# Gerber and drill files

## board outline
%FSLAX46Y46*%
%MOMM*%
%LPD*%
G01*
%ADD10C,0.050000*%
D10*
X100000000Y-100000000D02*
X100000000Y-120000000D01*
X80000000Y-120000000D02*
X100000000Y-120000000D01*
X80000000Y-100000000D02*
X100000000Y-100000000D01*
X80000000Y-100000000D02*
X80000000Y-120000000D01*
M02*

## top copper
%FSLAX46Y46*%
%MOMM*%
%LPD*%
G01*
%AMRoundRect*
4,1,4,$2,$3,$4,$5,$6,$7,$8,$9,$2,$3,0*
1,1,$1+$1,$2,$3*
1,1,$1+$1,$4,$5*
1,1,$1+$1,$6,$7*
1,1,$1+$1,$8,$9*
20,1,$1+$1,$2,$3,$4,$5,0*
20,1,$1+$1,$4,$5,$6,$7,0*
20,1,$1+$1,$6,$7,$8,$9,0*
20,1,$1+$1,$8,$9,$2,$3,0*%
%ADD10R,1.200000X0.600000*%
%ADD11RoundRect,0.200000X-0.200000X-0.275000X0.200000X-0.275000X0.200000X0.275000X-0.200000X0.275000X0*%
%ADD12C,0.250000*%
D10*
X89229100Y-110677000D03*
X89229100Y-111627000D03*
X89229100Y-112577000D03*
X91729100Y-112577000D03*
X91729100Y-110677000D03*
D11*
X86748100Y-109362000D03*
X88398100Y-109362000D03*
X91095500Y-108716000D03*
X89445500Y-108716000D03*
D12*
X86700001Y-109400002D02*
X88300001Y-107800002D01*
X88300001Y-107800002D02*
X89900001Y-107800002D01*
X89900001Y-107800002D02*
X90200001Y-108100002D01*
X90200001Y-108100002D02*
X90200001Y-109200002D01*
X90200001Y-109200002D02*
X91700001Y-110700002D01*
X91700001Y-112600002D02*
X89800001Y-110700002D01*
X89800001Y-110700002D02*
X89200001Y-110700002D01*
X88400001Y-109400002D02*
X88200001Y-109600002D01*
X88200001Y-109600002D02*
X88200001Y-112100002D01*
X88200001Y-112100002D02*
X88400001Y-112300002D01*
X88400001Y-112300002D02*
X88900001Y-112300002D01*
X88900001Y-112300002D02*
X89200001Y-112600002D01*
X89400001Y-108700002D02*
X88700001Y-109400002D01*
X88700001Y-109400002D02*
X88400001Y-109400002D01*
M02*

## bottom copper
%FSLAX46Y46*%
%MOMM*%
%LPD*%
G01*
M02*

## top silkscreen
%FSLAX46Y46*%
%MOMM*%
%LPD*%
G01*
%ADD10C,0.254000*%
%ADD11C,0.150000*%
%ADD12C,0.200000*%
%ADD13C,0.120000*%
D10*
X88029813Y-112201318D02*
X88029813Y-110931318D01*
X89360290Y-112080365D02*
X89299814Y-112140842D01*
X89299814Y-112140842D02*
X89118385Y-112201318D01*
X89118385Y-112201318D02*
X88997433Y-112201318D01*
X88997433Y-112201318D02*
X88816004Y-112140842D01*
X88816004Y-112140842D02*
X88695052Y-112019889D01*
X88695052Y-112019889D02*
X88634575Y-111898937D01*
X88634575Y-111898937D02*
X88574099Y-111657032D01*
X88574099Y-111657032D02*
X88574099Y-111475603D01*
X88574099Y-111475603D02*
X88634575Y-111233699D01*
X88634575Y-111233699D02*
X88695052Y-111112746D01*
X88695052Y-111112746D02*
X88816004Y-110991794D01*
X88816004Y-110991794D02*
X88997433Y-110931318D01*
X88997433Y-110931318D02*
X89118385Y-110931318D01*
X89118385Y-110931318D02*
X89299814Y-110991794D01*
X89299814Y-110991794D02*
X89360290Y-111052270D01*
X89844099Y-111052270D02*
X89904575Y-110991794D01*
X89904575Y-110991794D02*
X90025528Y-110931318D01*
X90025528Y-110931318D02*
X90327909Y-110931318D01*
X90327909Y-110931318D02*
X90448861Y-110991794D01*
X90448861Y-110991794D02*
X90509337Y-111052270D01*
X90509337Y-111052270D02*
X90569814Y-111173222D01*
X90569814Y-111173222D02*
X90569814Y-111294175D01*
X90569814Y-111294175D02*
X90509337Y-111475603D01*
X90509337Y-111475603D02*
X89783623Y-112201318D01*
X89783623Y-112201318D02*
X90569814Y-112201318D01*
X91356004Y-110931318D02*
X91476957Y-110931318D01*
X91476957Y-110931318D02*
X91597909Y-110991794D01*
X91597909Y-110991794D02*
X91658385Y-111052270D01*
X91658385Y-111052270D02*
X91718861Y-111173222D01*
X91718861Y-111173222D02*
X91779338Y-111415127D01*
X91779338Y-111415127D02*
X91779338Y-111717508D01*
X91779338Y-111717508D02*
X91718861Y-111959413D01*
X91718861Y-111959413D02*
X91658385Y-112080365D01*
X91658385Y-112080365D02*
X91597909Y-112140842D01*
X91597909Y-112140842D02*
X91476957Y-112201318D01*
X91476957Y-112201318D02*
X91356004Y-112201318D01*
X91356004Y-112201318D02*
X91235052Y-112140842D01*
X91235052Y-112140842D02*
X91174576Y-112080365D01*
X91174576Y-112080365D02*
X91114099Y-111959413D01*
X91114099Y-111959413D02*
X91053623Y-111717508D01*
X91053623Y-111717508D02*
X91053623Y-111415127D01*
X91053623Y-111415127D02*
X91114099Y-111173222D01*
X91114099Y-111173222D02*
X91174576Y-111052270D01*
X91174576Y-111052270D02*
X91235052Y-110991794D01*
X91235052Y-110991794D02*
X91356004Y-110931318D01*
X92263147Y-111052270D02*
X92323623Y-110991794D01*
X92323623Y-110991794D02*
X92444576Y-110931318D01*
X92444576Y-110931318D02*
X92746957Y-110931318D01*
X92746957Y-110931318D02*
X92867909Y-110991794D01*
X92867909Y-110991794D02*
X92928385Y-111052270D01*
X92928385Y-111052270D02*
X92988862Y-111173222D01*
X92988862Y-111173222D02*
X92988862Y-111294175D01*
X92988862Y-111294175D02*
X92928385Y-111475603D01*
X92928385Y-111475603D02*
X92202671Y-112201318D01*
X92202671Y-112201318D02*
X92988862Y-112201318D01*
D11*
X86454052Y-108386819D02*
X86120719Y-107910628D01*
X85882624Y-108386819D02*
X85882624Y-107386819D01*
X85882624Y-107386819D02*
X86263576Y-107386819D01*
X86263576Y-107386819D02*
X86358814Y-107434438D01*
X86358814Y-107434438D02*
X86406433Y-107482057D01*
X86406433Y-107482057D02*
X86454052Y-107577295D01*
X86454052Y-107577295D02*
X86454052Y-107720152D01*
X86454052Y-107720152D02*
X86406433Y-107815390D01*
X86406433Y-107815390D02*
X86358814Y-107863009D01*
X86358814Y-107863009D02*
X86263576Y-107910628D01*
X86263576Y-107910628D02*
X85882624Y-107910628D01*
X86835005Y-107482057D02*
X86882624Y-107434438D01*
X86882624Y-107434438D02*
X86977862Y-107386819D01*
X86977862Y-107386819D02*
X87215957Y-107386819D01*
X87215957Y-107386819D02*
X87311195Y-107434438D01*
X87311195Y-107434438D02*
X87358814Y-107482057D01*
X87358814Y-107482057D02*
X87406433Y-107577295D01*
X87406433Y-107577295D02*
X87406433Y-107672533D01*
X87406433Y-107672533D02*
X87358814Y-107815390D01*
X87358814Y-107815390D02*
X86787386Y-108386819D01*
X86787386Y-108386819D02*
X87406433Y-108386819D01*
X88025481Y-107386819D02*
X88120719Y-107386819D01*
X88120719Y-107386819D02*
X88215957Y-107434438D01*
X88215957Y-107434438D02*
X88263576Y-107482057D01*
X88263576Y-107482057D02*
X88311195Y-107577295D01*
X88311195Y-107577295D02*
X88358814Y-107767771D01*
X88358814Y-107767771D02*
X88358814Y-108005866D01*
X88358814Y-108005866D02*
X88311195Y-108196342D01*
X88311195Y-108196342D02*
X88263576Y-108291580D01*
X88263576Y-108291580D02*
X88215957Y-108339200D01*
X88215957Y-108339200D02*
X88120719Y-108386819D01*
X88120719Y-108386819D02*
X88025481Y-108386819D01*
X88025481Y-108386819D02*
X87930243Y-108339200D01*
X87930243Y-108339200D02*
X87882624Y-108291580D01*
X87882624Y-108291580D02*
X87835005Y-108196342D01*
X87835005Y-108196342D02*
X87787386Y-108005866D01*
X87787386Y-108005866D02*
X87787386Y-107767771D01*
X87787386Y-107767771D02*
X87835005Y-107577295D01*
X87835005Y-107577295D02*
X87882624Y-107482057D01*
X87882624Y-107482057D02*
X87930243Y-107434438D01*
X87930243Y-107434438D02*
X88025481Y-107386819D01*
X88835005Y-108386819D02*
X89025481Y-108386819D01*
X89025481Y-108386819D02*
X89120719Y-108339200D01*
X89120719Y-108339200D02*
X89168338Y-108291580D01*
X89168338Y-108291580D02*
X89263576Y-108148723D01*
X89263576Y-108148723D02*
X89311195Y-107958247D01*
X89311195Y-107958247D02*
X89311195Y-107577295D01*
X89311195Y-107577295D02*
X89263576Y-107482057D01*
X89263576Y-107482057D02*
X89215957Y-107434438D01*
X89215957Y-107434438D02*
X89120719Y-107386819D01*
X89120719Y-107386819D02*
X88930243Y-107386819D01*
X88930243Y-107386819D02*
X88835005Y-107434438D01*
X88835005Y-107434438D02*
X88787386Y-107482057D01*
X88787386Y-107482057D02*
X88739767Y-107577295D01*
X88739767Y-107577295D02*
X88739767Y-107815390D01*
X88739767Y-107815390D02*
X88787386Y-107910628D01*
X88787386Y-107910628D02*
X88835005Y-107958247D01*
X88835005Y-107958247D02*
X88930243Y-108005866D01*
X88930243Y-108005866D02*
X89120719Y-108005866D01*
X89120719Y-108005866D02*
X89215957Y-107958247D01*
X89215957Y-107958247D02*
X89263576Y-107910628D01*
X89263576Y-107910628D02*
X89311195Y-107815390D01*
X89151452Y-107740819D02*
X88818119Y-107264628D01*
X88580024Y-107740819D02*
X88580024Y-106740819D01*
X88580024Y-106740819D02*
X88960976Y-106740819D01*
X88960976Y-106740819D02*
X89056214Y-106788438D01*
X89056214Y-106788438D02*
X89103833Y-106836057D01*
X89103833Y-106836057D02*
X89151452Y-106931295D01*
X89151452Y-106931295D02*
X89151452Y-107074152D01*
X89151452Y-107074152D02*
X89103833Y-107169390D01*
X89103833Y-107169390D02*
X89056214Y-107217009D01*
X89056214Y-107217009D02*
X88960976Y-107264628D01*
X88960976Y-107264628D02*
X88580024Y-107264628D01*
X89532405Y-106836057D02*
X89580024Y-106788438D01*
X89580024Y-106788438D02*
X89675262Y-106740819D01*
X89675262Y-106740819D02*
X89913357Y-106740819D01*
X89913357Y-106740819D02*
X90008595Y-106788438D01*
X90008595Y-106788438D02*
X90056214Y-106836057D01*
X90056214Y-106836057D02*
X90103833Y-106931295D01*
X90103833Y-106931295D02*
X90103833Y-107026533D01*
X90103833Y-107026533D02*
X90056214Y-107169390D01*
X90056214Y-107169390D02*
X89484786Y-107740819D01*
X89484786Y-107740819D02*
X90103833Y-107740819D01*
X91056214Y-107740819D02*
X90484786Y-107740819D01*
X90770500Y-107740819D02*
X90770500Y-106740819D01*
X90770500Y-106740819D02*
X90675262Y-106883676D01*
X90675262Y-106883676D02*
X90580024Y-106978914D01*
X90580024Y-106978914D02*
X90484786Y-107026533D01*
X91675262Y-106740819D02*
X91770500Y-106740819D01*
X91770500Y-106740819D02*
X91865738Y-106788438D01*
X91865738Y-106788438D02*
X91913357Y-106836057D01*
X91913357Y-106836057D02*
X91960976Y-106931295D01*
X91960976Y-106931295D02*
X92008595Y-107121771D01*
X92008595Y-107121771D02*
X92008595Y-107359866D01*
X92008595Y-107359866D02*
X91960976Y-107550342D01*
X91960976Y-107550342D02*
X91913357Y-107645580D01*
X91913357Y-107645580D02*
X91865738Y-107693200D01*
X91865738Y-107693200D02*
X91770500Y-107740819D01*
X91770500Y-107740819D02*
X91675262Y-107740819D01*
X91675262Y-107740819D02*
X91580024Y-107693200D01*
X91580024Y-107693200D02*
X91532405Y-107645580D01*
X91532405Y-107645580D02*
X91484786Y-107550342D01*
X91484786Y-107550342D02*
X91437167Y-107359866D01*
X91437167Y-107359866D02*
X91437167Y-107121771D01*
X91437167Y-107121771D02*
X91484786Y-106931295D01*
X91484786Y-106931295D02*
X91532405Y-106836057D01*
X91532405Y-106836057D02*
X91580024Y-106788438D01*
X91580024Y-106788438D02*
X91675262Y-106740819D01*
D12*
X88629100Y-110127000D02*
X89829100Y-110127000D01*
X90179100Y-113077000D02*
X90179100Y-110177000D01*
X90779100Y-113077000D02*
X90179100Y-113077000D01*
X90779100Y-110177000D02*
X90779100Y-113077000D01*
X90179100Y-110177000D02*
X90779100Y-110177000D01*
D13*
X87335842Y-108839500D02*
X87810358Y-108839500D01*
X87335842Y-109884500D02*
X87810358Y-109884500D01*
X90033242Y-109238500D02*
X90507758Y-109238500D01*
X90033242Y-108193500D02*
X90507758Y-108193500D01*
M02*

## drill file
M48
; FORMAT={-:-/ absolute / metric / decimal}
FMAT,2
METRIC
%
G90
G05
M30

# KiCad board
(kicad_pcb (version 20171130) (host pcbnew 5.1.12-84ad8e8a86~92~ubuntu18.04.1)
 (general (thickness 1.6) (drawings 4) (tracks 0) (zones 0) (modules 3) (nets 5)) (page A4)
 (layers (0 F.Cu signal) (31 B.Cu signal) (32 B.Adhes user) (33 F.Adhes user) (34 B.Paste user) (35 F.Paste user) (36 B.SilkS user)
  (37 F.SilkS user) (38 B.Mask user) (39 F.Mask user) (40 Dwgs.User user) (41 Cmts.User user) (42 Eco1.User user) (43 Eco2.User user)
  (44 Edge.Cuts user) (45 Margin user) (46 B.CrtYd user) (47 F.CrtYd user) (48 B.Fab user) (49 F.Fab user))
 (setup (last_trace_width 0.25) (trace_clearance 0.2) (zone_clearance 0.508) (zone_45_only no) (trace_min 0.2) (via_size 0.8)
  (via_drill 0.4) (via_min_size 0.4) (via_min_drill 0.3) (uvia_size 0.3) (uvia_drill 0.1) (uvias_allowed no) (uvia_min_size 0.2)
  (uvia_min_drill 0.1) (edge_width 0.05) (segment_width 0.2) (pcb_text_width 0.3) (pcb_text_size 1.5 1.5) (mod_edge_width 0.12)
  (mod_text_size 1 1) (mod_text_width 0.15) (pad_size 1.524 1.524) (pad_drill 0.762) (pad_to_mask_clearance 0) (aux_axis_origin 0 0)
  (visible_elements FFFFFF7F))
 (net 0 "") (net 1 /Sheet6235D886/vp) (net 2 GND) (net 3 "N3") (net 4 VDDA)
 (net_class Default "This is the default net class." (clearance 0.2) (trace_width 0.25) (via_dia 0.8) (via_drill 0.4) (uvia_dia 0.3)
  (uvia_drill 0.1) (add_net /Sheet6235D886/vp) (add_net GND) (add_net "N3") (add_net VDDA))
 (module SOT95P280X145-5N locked (layer F.Cu) (at 90.479100 111.627000)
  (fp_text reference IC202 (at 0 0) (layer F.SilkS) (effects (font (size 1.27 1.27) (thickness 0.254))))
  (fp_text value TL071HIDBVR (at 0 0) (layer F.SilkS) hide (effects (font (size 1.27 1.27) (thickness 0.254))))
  (fp_line (start -1.85 -1.5) (end -0.65 -1.5) (layer F.SilkS) (width 0.2))
  (fp_line (start -0.3 1.45) (end -0.3 -1.45) (layer F.SilkS) (width 0.2))
  (fp_line (start 0.3 1.45) (end -0.3 1.45) (layer F.SilkS) (width 0.2))
  (fp_line (start 0.3 -1.45) (end 0.3 1.45) (layer F.SilkS) (width 0.2))
  (fp_line (start -0.3 -1.45) (end 0.3 -1.45) (layer F.SilkS) (width 0.2))
  (pad 1 smd rect (at -1.25 -0.95 90.000000) (size 0.6 1.2) (layers F.Cu F.Mask F.Paste) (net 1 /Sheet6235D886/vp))
  (pad 2 smd rect (at -1.25 0 90.000000) (size 0.6 1.2) (layers F.Cu F.Mask F.Paste) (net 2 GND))
  (pad 3 smd rect (at -1.25 0.95 90.000000) (size 0.6 1.2) (layers F.Cu F.Mask F.Paste) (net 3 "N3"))
  (pad 4 smd rect (at 1.25 0.95 90.000000) (size 0.6 1.2) (layers F.Cu F.Mask F.Paste) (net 1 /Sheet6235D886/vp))
  (pad 5 smd rect (at 1.25 -0.95 90.000000) (size 0.6 1.2) (layers F.Cu F.Mask F.Paste) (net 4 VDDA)))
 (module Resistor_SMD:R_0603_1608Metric (layer F.Cu) (at 87.573100 109.362000)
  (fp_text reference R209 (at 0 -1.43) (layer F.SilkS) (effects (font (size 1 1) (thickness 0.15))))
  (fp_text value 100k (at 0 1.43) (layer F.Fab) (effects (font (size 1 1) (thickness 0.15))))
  (fp_line (start -0.237258 -0.5225) (end 0.237258 -0.5225) (layer F.SilkS) (width 0.12))
  (fp_line (start -0.237258 0.5225) (end 0.237258 0.5225) (layer F.SilkS) (width 0.12))
  (pad 1 smd roundrect (at -0.825 0) (size 0.8 0.95) (layers F.Cu F.Mask F.Paste) (roundrect_rratio 0.25) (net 4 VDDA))
  (pad 2 smd roundrect (at 0.825 0) (size 0.8 0.95) (layers F.Cu F.Mask F.Paste) (roundrect_rratio 0.25) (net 3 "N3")))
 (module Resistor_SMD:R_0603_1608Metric (layer F.Cu) (at 90.270500 108.716000)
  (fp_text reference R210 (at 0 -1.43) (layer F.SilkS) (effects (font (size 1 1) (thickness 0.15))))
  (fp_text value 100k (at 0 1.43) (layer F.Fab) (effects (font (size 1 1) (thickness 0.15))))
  (fp_line (start -0.237258 0.5225) (end 0.237258 0.5225) (layer F.SilkS) (width 0.12))
  (fp_line (start -0.237258 -0.5225) (end 0.237258 -0.5225) (layer F.SilkS) (width 0.12))
  (pad 2 smd roundrect (at 0.825 0) (size 0.8 0.95) (layers F.Cu F.Mask F.Paste) (roundrect_rratio 0.25) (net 2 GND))
  (pad 1 smd roundrect (at -0.825 0) (size 0.8 0.95) (layers F.Cu F.Mask F.Paste) (roundrect_rratio 0.25) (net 3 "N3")))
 (gr_line (start 100 100) (end 100 120) (layer Edge.Cuts) (width 0.05))
 (gr_line (start 80 120) (end 100 120) (layer Edge.Cuts) (width 0.05))
 (gr_line (start 80 100) (end 100 100) (layer Edge.Cuts) (width 0.05))
 (gr_line (start 80 100) (end 80 120) (layer Edge.Cuts) (width 0.05))
 (segment (start 86.700001 109.400002) (end 88.300001 107.800002) (width 0.250000) (layer F.Cu) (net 4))
 (segment (start 88.300001 107.800002) (end 89.900001 107.800002) (width 0.250000) (layer F.Cu) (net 4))
 (segment (start 89.900001 107.800002) (end 90.200001 108.100002) (width 0.250000) (layer F.Cu) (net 4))
 (segment (start 90.200001 108.100002) (end 90.200001 109.200002) (width 0.250000) (layer F.Cu) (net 4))
 (segment (start 90.200001 109.200002) (end 91.700001 110.700002) (width 0.250000) (layer F.Cu) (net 4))
 (segment (start 91.700001 112.600002) (end 89.800001 110.700002) (width 0.250000) (layer F.Cu) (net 1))
 (segment (start 89.800001 110.700002) (end 89.200001 110.700002) (width 0.250000) (layer F.Cu) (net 1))
 (segment (start 88.400001 109.400002) (end 88.200001 109.600002) (width 0.250000) (layer F.Cu) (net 3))
 (segment (start 88.200001 109.600002) (end 88.200001 112.100002) (width 0.250000) (layer F.Cu) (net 3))
 (segment (start 88.200001 112.100002) (end 88.400001 112.300002) (width 0.250000) (layer F.Cu) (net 3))
 (segment (start 88.400001 112.300002) (end 88.900001 112.300002) (width 0.250000) (layer F.Cu) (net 3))
 (segment (start 88.900001 112.300002) (end 89.200001 112.600002) (width 0.250000) (layer F.Cu) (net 3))
 (segment (start 89.400001 108.700002) (end 88.700001 109.400002) (width 0.250000) (layer F.Cu) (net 3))
 (segment (start 88.700001 109.400002) (end 88.400001 109.400002) (width 0.250000) (layer F.Cu) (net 3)))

